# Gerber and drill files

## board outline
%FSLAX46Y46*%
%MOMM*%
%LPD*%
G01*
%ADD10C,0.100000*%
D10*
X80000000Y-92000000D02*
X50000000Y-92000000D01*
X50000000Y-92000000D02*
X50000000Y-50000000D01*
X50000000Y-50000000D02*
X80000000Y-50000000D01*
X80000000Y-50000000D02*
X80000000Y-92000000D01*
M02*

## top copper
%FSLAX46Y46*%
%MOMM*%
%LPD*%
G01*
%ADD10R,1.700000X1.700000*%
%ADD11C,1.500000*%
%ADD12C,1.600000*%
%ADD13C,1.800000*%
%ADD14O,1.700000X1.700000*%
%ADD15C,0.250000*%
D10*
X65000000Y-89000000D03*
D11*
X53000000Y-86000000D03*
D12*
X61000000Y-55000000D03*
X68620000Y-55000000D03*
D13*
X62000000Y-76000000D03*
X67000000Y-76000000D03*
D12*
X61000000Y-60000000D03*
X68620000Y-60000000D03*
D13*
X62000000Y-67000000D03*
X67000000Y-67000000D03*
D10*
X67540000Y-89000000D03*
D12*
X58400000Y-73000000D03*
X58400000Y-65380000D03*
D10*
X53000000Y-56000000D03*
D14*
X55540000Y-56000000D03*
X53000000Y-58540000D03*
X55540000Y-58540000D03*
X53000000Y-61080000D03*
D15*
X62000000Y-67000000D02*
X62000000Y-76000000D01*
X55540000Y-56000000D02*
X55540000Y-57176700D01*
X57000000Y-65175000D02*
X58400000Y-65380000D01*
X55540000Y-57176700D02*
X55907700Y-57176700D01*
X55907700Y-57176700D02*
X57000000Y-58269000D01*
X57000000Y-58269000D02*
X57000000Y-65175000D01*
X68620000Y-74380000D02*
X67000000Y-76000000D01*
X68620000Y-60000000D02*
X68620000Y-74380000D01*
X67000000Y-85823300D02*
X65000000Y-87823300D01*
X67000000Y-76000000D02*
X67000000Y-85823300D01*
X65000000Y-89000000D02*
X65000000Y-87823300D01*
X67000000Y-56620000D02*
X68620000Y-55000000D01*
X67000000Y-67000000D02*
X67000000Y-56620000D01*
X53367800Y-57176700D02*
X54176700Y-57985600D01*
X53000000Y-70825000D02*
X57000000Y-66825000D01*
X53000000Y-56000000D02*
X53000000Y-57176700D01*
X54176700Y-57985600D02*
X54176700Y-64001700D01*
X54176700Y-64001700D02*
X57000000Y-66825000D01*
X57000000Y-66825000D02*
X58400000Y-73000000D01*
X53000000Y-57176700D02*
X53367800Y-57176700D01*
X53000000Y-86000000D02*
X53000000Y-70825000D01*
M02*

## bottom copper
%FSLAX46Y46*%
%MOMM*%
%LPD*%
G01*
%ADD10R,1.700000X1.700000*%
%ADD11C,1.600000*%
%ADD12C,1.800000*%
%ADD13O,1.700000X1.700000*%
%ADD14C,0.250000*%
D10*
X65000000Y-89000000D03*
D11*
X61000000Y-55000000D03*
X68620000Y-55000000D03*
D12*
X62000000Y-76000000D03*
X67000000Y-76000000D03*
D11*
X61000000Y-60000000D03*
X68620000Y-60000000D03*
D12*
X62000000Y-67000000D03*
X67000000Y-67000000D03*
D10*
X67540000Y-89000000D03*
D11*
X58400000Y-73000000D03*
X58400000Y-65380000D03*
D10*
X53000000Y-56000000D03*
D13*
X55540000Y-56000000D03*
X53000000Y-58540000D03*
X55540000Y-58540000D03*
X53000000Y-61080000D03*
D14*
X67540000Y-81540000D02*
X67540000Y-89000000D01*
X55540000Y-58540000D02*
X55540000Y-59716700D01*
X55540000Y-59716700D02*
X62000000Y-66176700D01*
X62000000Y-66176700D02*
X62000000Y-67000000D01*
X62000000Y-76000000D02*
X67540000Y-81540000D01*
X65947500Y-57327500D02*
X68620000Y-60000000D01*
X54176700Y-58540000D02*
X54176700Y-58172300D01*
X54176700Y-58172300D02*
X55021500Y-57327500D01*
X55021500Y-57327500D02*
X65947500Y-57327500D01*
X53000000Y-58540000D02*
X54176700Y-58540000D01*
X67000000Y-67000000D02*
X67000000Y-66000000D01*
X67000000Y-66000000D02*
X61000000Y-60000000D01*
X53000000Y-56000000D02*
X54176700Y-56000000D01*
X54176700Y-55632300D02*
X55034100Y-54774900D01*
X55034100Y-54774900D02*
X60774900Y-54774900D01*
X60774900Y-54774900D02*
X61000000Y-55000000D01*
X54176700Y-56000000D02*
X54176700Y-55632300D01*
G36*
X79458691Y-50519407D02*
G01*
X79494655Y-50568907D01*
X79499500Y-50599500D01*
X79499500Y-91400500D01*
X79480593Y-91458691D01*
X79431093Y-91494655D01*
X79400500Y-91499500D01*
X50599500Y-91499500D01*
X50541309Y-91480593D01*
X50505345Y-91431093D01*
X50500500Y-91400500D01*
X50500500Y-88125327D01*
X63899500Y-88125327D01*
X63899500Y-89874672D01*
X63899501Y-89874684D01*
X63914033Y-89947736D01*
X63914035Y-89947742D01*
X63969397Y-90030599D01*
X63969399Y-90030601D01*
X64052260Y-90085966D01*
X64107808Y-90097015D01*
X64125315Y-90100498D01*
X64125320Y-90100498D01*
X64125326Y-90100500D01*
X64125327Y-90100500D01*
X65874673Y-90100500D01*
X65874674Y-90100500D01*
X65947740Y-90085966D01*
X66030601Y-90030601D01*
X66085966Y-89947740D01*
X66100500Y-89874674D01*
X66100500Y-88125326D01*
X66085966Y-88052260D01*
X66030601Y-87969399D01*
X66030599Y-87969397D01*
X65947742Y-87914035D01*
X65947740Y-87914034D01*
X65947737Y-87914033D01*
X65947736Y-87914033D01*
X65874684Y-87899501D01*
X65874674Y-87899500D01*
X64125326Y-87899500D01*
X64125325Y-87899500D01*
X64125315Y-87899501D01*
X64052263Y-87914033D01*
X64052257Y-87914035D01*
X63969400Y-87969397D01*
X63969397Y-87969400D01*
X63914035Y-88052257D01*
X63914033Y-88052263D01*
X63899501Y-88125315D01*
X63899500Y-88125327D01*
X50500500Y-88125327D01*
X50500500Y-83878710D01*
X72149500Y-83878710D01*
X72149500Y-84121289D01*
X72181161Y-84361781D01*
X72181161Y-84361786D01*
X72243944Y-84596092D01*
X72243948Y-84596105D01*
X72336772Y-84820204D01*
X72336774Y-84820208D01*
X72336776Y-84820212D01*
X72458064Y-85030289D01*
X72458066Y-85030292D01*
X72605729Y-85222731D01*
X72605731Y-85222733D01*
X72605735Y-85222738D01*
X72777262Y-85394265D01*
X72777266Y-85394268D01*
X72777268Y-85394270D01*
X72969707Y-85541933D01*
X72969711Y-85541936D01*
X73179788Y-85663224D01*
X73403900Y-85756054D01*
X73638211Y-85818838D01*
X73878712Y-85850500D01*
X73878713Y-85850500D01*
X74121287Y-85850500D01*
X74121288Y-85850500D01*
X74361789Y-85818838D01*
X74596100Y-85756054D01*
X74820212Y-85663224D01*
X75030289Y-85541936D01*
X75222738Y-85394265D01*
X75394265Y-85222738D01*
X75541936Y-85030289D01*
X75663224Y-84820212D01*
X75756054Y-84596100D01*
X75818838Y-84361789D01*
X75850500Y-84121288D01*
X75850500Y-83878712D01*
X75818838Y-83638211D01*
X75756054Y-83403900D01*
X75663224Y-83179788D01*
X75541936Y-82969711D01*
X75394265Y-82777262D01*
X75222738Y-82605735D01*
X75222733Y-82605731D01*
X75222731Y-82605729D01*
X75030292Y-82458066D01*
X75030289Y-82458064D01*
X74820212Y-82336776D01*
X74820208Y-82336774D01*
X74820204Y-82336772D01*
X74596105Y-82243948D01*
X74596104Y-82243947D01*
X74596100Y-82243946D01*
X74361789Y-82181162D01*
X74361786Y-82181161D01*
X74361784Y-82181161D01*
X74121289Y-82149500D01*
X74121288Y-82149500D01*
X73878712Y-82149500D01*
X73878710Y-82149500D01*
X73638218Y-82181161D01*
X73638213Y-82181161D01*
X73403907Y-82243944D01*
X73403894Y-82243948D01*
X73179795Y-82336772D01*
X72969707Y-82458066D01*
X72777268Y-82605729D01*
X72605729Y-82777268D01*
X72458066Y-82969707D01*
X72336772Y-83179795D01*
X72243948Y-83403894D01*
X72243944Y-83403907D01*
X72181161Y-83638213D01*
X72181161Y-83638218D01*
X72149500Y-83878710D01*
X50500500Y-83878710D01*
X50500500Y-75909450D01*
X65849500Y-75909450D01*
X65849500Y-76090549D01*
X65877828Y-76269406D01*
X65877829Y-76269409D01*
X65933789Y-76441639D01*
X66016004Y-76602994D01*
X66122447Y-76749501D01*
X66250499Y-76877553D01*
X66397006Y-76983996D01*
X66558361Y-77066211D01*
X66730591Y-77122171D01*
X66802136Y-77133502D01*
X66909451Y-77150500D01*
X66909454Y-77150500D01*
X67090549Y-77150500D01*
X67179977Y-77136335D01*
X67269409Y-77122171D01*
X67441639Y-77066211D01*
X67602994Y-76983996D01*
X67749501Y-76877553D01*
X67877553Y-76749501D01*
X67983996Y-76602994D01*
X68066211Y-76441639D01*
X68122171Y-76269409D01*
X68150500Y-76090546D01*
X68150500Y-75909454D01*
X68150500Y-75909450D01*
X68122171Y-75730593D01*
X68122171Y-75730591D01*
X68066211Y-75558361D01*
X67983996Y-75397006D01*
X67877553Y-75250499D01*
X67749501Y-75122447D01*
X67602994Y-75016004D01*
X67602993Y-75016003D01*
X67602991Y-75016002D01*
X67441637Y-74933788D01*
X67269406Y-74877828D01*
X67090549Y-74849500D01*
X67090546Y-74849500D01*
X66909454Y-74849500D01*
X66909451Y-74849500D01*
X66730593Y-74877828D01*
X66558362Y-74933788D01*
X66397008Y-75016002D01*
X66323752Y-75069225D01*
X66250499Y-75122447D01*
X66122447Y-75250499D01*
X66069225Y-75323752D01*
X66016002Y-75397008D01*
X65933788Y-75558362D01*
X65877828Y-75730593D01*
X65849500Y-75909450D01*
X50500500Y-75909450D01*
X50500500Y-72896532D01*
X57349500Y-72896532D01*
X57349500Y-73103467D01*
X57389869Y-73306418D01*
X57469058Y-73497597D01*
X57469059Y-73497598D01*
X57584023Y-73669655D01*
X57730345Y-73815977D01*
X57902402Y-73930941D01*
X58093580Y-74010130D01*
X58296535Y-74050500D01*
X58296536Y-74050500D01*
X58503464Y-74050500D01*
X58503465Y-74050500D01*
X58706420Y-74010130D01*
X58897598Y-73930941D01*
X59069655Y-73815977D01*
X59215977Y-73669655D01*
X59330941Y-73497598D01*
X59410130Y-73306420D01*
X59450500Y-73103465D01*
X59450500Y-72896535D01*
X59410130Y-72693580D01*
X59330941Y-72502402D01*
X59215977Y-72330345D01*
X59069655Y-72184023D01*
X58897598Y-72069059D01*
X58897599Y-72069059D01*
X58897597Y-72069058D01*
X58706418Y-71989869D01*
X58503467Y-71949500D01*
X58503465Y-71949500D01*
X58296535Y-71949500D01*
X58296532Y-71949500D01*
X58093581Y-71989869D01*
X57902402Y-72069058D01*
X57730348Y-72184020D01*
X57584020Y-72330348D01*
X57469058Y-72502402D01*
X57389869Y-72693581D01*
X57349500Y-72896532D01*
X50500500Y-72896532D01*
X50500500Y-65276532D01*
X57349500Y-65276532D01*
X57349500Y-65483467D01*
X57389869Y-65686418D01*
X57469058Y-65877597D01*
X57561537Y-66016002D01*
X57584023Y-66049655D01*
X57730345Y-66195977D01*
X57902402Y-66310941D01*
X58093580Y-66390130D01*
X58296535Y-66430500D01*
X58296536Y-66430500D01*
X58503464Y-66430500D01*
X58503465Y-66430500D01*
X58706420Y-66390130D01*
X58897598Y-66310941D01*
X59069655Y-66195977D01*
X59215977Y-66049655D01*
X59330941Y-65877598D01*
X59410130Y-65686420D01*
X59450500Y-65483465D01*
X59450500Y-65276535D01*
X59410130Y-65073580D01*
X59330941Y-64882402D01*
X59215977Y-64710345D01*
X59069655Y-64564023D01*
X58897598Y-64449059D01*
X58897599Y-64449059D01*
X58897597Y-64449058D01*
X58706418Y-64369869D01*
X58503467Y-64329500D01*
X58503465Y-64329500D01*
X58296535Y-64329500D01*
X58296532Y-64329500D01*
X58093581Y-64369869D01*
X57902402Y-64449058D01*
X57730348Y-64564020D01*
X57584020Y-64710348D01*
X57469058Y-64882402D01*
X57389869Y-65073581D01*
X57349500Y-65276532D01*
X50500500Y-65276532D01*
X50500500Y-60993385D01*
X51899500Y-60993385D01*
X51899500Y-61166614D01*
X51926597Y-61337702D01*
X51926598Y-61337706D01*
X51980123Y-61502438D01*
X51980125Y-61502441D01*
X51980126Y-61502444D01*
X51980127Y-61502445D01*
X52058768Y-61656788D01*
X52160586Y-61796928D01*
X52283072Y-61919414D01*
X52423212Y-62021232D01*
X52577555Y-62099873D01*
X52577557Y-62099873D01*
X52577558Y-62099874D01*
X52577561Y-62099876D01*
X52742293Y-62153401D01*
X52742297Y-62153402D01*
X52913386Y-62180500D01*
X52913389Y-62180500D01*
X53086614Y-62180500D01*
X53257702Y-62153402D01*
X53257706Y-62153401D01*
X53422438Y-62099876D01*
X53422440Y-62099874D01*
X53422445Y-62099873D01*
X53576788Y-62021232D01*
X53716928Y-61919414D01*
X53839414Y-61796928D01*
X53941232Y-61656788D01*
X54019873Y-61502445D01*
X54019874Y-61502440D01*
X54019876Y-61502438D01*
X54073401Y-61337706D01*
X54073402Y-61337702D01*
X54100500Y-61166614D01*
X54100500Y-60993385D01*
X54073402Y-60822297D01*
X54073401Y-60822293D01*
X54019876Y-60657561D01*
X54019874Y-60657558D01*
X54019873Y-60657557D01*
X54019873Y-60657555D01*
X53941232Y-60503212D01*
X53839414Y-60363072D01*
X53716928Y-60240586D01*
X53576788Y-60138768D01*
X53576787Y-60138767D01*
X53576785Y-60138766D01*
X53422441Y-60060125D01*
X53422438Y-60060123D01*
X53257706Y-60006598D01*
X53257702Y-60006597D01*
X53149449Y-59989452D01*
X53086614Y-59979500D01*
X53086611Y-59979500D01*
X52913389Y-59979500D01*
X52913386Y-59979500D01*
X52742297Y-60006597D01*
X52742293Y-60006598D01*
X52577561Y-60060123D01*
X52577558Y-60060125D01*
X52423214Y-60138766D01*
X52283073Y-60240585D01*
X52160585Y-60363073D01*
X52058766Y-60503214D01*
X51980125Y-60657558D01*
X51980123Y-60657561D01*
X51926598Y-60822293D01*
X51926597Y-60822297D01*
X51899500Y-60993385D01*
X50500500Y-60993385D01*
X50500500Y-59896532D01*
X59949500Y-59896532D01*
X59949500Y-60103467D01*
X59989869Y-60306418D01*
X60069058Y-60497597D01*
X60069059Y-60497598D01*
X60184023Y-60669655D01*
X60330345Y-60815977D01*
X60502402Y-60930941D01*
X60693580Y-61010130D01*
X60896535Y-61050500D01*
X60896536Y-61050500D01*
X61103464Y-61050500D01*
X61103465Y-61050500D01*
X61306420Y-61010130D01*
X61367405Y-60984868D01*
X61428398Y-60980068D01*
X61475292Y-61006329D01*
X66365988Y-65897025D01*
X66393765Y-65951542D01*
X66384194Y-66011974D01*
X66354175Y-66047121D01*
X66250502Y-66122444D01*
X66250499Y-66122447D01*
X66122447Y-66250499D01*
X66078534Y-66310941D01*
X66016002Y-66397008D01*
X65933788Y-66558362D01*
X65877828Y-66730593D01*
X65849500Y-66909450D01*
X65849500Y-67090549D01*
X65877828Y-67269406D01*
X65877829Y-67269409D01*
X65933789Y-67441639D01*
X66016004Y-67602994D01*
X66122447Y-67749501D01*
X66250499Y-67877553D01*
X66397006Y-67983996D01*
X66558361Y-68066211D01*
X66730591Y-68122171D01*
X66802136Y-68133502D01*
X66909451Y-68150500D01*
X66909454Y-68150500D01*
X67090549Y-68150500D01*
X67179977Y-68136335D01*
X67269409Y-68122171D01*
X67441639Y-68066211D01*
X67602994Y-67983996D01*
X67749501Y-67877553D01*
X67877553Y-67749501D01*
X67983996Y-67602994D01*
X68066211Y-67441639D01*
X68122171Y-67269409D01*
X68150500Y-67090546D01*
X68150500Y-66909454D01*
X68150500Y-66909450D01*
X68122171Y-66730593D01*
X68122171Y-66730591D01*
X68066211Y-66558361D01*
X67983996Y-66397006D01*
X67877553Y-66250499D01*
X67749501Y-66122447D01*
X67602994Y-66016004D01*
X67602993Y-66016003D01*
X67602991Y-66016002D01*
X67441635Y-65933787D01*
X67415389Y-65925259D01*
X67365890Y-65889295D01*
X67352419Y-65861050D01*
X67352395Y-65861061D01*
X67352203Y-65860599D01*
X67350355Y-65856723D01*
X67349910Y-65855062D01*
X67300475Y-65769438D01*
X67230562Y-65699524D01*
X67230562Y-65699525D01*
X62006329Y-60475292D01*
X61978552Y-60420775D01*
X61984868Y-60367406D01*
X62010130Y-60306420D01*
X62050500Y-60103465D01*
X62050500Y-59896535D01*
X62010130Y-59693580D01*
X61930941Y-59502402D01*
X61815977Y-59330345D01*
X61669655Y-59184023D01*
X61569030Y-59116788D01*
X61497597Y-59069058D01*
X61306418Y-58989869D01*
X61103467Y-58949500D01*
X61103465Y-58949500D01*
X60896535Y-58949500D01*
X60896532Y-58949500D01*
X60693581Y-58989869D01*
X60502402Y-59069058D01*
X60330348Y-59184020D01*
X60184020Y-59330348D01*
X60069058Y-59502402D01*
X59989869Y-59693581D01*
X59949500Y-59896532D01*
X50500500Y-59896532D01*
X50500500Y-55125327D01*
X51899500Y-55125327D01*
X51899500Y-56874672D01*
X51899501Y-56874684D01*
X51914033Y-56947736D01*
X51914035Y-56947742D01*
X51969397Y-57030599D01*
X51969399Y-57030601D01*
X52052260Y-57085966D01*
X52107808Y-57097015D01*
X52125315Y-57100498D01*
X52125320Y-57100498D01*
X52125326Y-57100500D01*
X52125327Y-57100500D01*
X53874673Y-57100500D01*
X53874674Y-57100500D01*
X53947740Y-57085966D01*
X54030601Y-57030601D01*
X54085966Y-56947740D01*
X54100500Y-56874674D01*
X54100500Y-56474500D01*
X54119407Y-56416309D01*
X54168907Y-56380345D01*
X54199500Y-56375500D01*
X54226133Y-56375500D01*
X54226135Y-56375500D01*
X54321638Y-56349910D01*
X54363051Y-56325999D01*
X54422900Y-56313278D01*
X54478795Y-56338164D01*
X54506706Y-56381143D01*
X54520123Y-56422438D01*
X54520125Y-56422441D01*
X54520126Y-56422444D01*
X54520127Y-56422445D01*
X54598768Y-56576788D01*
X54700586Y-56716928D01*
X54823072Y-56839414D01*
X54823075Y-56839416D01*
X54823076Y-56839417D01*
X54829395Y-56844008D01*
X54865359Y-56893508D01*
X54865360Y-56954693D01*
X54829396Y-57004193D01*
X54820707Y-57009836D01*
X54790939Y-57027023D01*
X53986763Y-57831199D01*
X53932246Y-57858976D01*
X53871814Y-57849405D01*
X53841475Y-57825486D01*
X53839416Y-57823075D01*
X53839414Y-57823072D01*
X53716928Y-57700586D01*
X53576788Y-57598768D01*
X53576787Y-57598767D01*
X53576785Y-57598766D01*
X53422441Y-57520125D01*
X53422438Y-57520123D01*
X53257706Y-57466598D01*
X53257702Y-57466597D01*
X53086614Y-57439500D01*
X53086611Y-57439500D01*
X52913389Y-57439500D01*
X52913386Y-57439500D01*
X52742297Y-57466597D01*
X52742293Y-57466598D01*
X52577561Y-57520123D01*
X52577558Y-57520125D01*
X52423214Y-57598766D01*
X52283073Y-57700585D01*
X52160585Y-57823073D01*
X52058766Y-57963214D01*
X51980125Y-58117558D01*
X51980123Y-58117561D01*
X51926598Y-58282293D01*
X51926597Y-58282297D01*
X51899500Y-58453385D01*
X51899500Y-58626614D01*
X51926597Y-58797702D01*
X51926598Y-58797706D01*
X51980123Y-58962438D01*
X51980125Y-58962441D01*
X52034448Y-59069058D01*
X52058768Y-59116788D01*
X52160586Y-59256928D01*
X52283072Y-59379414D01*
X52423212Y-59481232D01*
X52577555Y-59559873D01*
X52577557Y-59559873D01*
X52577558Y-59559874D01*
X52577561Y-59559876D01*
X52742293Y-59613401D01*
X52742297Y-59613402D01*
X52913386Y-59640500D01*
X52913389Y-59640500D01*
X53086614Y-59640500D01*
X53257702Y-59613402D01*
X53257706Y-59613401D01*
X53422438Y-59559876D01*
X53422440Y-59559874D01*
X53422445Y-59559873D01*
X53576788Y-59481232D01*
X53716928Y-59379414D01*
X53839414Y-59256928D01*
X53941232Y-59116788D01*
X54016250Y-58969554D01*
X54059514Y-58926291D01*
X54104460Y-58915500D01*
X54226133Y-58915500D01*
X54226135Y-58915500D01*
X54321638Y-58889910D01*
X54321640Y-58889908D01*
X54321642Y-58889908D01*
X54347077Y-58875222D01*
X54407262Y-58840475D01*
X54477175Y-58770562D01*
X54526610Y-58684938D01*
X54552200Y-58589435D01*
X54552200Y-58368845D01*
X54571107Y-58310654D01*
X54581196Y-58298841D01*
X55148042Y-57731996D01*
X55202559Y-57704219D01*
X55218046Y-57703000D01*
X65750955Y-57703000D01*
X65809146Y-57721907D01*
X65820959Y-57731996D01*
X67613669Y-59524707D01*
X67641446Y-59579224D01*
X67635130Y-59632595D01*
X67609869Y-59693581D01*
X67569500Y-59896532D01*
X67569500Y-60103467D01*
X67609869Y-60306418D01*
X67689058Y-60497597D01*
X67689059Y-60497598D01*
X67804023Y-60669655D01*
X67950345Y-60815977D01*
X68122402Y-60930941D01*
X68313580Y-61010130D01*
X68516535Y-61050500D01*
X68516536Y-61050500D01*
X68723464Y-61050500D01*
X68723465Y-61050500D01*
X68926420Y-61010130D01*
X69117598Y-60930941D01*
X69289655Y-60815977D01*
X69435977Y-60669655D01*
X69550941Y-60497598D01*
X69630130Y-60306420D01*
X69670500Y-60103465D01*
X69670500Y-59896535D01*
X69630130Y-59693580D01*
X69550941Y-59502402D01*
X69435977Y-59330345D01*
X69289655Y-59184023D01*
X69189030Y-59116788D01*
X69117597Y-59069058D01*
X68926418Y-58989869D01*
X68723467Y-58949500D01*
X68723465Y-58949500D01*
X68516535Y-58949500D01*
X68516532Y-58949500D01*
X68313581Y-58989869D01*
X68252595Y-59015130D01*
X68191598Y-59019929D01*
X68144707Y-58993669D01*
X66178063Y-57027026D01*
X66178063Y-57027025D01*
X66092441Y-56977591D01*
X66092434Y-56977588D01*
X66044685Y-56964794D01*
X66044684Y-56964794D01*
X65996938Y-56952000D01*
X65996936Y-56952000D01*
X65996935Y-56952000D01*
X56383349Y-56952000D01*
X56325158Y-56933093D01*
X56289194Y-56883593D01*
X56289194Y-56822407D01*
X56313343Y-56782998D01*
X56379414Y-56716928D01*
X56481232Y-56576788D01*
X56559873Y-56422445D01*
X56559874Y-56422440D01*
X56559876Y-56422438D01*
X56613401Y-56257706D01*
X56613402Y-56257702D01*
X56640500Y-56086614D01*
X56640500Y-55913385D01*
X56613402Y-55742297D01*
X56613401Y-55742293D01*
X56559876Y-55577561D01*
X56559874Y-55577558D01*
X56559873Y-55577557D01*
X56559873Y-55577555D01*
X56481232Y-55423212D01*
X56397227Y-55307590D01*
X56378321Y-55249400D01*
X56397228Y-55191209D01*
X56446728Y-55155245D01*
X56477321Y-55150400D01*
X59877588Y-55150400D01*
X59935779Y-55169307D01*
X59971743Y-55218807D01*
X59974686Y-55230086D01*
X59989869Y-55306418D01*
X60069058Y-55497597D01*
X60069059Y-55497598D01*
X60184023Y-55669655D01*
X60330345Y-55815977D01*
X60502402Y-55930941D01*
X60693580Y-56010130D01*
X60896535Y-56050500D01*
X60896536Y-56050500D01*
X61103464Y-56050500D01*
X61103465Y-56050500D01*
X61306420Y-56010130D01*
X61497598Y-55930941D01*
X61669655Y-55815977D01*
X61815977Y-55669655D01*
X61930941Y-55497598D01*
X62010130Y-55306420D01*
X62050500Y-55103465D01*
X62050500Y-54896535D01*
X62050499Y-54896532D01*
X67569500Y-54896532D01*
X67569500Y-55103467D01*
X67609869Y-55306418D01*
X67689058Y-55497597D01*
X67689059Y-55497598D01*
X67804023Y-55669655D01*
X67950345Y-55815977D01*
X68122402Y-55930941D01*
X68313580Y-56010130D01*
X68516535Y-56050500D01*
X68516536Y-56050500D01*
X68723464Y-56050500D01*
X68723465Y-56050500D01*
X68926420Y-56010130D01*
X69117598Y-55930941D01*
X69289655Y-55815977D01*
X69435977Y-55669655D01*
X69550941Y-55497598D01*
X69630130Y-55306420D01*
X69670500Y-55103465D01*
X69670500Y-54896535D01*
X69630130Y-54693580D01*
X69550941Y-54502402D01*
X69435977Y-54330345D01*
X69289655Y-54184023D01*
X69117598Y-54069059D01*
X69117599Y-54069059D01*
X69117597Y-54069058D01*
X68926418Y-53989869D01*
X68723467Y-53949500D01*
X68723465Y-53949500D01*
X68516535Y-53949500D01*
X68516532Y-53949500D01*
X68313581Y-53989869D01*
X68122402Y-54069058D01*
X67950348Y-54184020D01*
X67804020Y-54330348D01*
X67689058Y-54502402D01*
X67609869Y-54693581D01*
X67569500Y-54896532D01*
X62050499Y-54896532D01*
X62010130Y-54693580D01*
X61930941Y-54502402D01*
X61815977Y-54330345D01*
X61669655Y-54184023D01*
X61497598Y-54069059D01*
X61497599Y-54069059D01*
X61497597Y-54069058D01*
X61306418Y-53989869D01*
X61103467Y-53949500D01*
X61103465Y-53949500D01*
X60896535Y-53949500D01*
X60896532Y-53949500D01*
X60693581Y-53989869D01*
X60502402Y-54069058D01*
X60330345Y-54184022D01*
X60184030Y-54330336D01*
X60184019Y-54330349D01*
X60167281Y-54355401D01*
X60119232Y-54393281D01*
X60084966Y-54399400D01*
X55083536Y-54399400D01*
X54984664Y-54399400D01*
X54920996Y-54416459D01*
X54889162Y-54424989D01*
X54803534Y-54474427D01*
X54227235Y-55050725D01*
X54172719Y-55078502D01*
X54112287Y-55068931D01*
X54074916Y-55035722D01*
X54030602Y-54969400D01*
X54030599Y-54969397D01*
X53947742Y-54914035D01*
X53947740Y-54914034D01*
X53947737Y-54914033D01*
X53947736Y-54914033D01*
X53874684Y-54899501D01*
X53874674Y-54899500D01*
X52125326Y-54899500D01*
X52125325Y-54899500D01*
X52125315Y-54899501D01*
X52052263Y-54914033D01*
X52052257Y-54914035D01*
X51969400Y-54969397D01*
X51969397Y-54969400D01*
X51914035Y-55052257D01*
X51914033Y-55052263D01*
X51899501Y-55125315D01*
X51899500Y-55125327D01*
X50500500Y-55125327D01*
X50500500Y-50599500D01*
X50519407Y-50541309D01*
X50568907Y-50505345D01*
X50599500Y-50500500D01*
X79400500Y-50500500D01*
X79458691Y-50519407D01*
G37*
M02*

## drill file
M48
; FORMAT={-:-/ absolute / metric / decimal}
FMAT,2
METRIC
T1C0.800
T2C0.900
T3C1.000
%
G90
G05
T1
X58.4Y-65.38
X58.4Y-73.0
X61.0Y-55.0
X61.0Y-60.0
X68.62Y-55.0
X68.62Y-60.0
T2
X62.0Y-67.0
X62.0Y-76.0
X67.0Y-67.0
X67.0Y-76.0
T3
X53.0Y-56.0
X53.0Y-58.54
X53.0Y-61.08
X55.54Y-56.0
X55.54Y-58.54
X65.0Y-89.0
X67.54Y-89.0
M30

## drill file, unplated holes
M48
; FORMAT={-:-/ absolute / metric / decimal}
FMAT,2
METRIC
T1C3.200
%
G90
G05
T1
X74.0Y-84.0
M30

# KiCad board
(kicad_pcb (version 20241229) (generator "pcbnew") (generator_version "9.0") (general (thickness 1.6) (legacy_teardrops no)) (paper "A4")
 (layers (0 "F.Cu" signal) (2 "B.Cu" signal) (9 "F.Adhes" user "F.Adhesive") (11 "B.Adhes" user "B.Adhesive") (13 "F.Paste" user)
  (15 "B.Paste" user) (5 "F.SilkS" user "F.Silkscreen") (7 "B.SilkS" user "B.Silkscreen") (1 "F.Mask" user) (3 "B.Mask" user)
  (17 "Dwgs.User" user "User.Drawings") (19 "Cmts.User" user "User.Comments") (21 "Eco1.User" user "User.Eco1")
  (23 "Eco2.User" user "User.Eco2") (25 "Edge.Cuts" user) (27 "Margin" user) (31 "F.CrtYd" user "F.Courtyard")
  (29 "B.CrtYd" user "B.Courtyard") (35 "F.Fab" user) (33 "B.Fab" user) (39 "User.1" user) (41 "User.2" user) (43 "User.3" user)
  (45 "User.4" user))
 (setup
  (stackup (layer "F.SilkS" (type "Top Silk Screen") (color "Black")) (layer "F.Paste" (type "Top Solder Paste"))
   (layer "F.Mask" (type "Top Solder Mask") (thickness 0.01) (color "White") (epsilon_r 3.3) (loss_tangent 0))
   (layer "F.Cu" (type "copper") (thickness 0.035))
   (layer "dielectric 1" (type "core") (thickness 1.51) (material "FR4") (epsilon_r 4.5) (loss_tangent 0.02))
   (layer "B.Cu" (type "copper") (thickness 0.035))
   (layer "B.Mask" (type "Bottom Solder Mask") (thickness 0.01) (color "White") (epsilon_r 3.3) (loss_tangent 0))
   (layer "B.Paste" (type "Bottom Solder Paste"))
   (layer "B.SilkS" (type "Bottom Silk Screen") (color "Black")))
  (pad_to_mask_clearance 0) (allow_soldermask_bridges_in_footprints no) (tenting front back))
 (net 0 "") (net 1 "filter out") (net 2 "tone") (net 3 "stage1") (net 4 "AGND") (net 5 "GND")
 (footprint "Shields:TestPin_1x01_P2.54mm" (layer "F.Cu") (at 65 89)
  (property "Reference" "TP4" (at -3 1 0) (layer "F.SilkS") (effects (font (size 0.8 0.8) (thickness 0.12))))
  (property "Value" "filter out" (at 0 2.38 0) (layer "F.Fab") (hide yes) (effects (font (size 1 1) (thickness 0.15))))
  (pad "1" thru_hole rect (at 0 0) (size 1.7 1.7) (drill 1) (layers "*.Cu" "*.Mask") (remove_unused_layers no) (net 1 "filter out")))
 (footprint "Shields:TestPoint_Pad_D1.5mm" (layer "F.Cu") (at 53 86)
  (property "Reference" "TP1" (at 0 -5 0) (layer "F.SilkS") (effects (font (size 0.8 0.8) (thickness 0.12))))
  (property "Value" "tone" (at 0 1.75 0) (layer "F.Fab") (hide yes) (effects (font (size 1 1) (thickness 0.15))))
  (pad "1" smd circle (at 0 0) (size 1.5 1.5) (layers "F.Cu" "F.Mask") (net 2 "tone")))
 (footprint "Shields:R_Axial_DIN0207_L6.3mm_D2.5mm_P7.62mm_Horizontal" (layer "F.Cu") (at 61 55)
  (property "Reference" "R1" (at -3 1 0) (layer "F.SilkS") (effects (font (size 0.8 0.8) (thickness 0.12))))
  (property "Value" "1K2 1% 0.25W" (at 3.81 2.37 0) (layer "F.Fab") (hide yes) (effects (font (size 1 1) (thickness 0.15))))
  (pad "1" thru_hole circle (at 0 0) (size 1.6 1.6) (drill 0.8) (layers "*.Cu" "*.Mask") (remove_unused_layers no) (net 2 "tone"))
  (pad "2" thru_hole circle (at 7.62 0) (size 1.6 1.6) (drill 0.8) (layers "*.Cu" "*.Mask") (remove_unused_layers no) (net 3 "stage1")))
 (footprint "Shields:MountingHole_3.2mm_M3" (layer "F.Cu") (at 74 84)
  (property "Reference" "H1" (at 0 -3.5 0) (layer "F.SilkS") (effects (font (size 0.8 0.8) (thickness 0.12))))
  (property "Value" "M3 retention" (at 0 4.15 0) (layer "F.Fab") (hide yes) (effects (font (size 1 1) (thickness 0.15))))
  (pad "" np_thru_hole circle (at 0 0) (size 3.2 3.2) (drill 3.2) (layers "*.Cu" "*.Mask")))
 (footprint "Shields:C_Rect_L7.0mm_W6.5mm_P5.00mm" (layer "F.Cu") (at 62 76)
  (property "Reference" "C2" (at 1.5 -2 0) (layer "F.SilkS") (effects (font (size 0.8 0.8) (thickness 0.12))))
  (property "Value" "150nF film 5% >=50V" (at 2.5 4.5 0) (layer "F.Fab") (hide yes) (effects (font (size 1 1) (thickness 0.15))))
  (pad "1" thru_hole circle (at 0 0) (size 1.8 1.8) (drill 0.9) (layers "*.Cu" "*.Mask") (remove_unused_layers no) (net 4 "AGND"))
  (pad "2" thru_hole circle (at 5 0) (size 1.8 1.8) (drill 0.9) (layers "*.Cu" "*.Mask") (remove_unused_layers no) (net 1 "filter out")))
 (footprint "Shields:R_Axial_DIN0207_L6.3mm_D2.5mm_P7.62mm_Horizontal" (layer "F.Cu") (at 61 60)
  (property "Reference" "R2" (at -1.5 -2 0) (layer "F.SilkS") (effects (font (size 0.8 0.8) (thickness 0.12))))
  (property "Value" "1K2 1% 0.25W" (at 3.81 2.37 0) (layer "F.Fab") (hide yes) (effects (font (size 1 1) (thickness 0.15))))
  (pad "1" thru_hole circle (at 0 0) (size 1.6 1.6) (drill 0.8) (layers "*.Cu" "*.Mask") (remove_unused_layers no) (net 3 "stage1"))
  (pad "2" thru_hole circle (at 7.62 0) (size 1.6 1.6) (drill 0.8) (layers "*.Cu" "*.Mask") (remove_unused_layers no) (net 1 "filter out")))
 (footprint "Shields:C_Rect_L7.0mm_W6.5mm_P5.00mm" (layer "F.Cu") (at 62 67)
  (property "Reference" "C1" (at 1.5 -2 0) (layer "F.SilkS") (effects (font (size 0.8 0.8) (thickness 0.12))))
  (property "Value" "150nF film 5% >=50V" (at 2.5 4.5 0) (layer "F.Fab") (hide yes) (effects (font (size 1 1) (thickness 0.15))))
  (pad "1" thru_hole circle (at 0 0) (size 1.8 1.8) (drill 0.9) (layers "*.Cu" "*.Mask") (remove_unused_layers no) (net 4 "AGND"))
  (pad "2" thru_hole circle (at 5 0) (size 1.8 1.8) (drill 0.9) (layers "*.Cu" "*.Mask") (remove_unused_layers no) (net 3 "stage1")))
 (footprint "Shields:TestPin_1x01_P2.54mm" (layer "F.Cu") (at 67.54 89)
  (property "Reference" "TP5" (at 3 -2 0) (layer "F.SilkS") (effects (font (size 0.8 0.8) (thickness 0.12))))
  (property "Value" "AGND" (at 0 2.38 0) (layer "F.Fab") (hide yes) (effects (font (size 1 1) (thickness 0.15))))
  (pad "1" thru_hole rect (at 0 0) (size 1.7 1.7) (drill 1) (layers "*.Cu" "*.Mask") (remove_unused_layers no) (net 4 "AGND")))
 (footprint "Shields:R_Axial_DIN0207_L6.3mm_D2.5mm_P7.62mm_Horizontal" (layer "F.Cu") (at 58.4 73 90)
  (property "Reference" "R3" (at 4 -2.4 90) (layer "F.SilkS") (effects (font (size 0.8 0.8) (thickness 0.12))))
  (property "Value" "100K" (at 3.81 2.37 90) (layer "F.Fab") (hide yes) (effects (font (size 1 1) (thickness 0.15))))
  (pad "1" thru_hole circle (at 0 0 90) (size 1.6 1.6) (drill 0.8) (layers "*.Cu" "*.Mask") (remove_unused_layers no) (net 2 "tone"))
  (pad "2" thru_hole circle (at 7.62 0 90) (size 1.6 1.6) (drill 0.8) (layers "*.Cu" "*.Mask") (remove_unused_layers no) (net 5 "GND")))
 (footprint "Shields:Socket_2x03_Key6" (layer "B.Cu") (at 53 56)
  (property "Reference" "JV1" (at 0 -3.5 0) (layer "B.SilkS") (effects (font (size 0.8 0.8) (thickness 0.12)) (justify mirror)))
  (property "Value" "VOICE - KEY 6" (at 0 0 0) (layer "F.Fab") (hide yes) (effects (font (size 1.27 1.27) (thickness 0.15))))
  (pad "1" thru_hole rect (at 0 0) (size 1.7 1.7) (drill 1) (layers "*.Cu" "*.Mask") (remove_unused_layers no) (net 2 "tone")
   (thermal_bridge_angle 45))
  (pad "2" thru_hole oval (at 2.54 0) (size 1.7 1.7) (drill 1) (layers "*.Cu" "*.Mask") (remove_unused_layers no) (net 5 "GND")
   (thermal_bridge_angle 45))
  (pad "3" thru_hole oval (at 0 2.54) (size 1.7 1.7) (drill 1) (layers "*.Cu" "*.Mask") (remove_unused_layers no) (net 1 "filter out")
   (thermal_bridge_angle 45))
  (pad "4" thru_hole oval (at 2.54 2.54) (size 1.7 1.7) (drill 1) (layers "*.Cu" "*.Mask") (remove_unused_layers no) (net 4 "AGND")
   (thermal_bridge_angle 45))
  (pad "5" thru_hole oval (at 0 5.08) (size 1.7 1.7) (drill 1) (layers "*.Cu" "*.Mask") (remove_unused_layers no) (thermal_bridge_angle 45)))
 (gr_line (start 80 92) (end 50 92) (stroke (width 0.1) (type default)) (layer "Edge.Cuts"))
 (gr_line (start 50 92) (end 50 50) (stroke (width 0.1) (type default)) (layer "Edge.Cuts"))
 (gr_line (start 50 50) (end 80 50) (stroke (width 0.1) (type default)) (layer "Edge.Cuts"))
 (gr_line (start 80 50) (end 80 92) (stroke (width 0.1) (type default)) (layer "Edge.Cuts"))
 (segment (start 62 67) (end 62 76) (width 0.25) (layer "F.Cu") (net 4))
 (segment (start 67.54 81.54) (end 67.54 89) (width 0.25) (layer "B.Cu") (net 4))
 (segment (start 55.54 58.54) (end 55.54 59.7167) (width 0.25) (layer "B.Cu") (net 4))
 (segment (start 55.54 59.7167) (end 62 66.1767) (width 0.25) (layer "B.Cu") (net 4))
 (segment (start 62 66.1767) (end 62 67) (width 0.25) (layer "B.Cu") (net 4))
 (segment (start 62 76) (end 67.54 81.54) (width 0.25) (layer "B.Cu") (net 4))
 (segment (start 55.54 56) (end 55.54 57.1767) (width 0.25) (layer "F.Cu") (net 5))
 (segment (start 57 65.175) (end 58.4 65.38) (width 0.25) (layer "F.Cu") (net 5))
 (segment (start 55.54 57.1767) (end 55.9077 57.1767) (width 0.25) (layer "F.Cu") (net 5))
 (segment (start 55.9077 57.1767) (end 57 58.269) (width 0.25) (layer "F.Cu") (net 5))
 (segment (start 57 58.269) (end 57 65.175) (width 0.25) (layer "F.Cu") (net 5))
 (segment (start 68.62 74.38) (end 67 76) (width 0.25) (layer "F.Cu") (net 1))
 (segment (start 68.62 60) (end 68.62 74.38) (width 0.25) (layer "F.Cu") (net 1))
 (segment (start 67 85.8233) (end 65 87.8233) (width 0.25) (layer "F.Cu") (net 1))
 (segment (start 67 76) (end 67 85.8233) (width 0.25) (layer "F.Cu") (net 1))
 (segment (start 65 89) (end 65 87.8233) (width 0.25) (layer "F.Cu") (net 1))
 (segment (start 65.9475 57.3275) (end 68.62 60) (width 0.25) (layer "B.Cu") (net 1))
 (segment (start 54.1767 58.54) (end 54.1767 58.1723) (width 0.25) (layer "B.Cu") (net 1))
 (segment (start 54.1767 58.1723) (end 55.0215 57.3275) (width 0.25) (layer "B.Cu") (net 1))
 (segment (start 55.0215 57.3275) (end 65.9475 57.3275) (width 0.25) (layer "B.Cu") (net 1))
 (segment (start 53 58.54) (end 54.1767 58.54) (width 0.25) (layer "B.Cu") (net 1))
 (segment (start 67 56.62) (end 68.62 55) (width 0.25) (layer "F.Cu") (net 3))
 (segment (start 67 67) (end 67 56.62) (width 0.25) (layer "F.Cu") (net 3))
 (segment (start 67 67) (end 67 66) (width 0.25) (layer "B.Cu") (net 3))
 (segment (start 67 66) (end 61 60) (width 0.25) (layer "B.Cu") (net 3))
 (segment (start 53.3678 57.1767) (end 54.1767 57.9856) (width 0.25) (layer "F.Cu") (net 2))
 (segment (start 53 70.825) (end 57 66.825) (width 0.25) (layer "F.Cu") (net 2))
 (segment (start 53 56) (end 53 57.1767) (width 0.25) (layer "F.Cu") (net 2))
 (segment (start 54.1767 57.9856) (end 54.1767 64.0017) (width 0.25) (layer "F.Cu") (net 2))
 (segment (start 54.1767 64.0017) (end 57 66.825) (width 0.25) (layer "F.Cu") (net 2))
 (segment (start 57 66.825) (end 58.4 73) (width 0.25) (layer "F.Cu") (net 2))
 (segment (start 53 57.1767) (end 53.3678 57.1767) (width 0.25) (layer "F.Cu") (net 2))
 (segment (start 53 86) (end 53 70.825) (width 0.25) (layer "F.Cu") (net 2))
 (segment (start 53 56) (end 54.1767 56) (width 0.25) (layer "B.Cu") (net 2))
 (segment (start 54.1767 55.6323) (end 55.0341 54.7749) (width 0.25) (layer "B.Cu") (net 2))
 (segment (start 55.0341 54.7749) (end 60.7749 54.7749) (width 0.25) (layer "B.Cu") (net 2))
 (segment (start 60.7749 54.7749) (end 61 55) (width 0.25) (layer "B.Cu") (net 2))
 (segment (start 54.1767 56) (end 54.1767 55.6323) (width 0.25) (layer "B.Cu") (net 2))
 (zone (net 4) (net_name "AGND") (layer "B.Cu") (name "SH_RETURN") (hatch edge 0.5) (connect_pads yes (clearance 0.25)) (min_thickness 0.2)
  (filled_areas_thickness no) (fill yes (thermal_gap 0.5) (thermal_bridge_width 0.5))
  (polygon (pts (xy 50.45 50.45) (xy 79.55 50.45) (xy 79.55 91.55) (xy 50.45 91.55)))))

